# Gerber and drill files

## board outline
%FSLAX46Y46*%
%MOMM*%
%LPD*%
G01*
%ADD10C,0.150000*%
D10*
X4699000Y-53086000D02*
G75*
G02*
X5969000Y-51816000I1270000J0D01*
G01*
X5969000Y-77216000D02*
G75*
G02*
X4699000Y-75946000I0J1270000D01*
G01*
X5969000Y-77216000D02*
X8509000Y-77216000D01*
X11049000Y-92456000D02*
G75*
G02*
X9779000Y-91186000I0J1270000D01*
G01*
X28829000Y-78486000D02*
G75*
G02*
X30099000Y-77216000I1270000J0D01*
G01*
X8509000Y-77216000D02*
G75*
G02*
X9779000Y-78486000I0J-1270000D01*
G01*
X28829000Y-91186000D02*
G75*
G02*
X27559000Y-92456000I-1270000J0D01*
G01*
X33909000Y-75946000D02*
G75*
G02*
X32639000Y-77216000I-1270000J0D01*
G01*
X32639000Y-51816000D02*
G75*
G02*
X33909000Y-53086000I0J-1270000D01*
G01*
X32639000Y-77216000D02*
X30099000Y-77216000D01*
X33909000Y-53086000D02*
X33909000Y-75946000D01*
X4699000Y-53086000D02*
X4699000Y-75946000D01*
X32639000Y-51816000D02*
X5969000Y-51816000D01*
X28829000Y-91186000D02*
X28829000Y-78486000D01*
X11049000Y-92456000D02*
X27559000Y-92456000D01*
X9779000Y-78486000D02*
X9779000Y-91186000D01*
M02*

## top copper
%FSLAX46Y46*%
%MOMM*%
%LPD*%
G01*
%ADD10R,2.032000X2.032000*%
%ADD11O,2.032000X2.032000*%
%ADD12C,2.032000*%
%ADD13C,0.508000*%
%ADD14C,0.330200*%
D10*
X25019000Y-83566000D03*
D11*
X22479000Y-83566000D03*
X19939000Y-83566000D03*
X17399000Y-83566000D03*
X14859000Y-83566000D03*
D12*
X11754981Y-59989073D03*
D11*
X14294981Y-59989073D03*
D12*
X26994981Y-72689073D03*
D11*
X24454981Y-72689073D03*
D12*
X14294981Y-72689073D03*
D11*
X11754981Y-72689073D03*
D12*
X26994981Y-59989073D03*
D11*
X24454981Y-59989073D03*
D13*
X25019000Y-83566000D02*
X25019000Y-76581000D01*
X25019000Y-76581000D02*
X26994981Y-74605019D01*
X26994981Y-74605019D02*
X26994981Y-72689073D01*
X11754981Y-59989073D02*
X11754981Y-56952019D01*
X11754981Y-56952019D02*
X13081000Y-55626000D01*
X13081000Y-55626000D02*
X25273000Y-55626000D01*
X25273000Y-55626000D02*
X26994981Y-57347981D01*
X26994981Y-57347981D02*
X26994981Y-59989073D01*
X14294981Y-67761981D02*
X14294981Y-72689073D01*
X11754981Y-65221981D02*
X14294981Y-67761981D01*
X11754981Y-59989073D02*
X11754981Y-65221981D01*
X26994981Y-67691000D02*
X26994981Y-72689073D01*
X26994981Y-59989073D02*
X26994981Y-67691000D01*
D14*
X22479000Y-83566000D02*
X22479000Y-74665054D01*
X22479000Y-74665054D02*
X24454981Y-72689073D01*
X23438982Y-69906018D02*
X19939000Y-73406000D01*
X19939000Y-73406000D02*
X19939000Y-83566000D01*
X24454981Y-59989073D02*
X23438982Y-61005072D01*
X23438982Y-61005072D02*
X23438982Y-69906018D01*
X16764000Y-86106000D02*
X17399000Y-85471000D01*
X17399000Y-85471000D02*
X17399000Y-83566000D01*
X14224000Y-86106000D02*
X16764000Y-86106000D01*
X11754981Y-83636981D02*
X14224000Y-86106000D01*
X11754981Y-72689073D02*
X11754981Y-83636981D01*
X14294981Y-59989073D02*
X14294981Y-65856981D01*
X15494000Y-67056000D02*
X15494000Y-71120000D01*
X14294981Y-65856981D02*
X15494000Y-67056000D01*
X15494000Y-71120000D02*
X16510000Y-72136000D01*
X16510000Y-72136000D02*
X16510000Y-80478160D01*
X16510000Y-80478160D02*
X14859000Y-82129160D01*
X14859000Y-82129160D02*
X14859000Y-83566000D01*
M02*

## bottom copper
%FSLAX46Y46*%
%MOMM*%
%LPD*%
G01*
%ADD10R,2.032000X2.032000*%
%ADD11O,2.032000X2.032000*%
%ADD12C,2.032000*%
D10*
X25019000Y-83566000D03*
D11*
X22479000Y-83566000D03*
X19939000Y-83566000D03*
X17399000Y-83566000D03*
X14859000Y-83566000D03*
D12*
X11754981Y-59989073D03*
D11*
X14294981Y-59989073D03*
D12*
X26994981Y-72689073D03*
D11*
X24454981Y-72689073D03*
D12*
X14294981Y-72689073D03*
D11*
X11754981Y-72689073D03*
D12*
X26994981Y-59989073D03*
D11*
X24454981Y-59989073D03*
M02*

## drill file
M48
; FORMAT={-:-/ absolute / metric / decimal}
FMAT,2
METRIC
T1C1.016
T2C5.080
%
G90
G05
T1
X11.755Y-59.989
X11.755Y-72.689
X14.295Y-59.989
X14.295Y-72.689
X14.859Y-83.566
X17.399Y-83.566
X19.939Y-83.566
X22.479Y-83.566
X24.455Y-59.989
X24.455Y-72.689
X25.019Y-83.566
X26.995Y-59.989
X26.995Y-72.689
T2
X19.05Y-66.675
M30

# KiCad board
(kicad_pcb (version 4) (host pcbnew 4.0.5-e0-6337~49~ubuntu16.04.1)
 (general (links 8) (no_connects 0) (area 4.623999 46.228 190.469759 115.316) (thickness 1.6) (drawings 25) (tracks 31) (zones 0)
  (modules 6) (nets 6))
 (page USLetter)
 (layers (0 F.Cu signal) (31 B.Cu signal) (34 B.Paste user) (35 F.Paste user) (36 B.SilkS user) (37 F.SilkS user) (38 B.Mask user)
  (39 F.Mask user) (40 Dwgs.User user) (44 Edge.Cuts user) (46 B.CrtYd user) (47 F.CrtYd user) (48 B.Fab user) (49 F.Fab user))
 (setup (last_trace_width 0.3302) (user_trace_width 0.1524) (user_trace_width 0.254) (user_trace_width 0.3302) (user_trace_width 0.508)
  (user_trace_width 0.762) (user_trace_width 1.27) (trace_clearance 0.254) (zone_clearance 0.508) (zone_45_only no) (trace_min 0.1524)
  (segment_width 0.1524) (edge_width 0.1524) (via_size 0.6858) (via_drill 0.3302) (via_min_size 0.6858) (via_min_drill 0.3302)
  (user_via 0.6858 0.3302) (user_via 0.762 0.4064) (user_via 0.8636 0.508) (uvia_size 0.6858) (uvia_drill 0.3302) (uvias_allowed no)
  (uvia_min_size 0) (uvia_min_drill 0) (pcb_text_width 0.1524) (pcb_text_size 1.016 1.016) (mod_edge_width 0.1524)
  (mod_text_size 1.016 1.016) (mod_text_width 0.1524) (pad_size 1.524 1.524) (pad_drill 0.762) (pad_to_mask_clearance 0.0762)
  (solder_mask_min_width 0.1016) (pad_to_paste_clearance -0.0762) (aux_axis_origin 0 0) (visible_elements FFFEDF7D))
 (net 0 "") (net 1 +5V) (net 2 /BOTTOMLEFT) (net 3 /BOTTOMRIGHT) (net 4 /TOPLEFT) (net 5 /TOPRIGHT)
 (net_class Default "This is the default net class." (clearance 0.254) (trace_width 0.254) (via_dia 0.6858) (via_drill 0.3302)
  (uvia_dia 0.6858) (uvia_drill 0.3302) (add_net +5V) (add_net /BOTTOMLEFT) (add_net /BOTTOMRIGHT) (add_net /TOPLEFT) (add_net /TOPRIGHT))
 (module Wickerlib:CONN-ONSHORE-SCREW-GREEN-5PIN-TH (layer F.Cu) (at 25.019 83.566 270)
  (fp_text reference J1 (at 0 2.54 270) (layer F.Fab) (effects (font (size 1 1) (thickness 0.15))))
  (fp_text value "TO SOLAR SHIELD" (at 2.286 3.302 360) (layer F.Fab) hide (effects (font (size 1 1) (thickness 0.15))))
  (pad 1 thru_hole rect (at 0 0 270) (size 2.032 2.032) (drill 1.016) (layers *.Cu *.Mask F.SilkS) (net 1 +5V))
  (pad 2 thru_hole oval (at 0 2.54 270) (size 2.032 2.032) (drill 1.016) (layers *.Cu *.Mask F.SilkS) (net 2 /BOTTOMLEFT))
  (pad 3 thru_hole oval (at 0 5.08 270) (size 2.032 2.032) (drill 1.016) (layers *.Cu *.Mask F.SilkS) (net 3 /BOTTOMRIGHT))
  (pad 4 thru_hole oval (at 0 7.62 270) (size 2.032 2.032) (drill 1.016) (layers *.Cu *.Mask F.SilkS) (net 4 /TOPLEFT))
  (pad 5 thru_hole oval (at 0 10.16 270) (size 2.032 2.032) (drill 1.016) (layers *.Cu *.Mask F.SilkS) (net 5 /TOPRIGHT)))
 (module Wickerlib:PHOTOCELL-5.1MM (layer F.Cu) (at 13.024981 59.989073 90)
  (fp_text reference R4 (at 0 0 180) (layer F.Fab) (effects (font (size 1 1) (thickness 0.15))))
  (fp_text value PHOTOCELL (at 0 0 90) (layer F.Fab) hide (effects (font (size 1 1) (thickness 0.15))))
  (pad 1 thru_hole circle (at 0 -1.27 90) (size 2.032 2.032) (drill 1.016) (layers *.Cu *.Mask F.SilkS) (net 1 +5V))
  (pad 2 thru_hole oval (at 0 1.27 90) (size 2.032 2.032) (drill 1.016) (layers *.Cu *.Mask F.SilkS) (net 5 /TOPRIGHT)))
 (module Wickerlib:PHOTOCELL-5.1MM (layer F.Cu) (at 25.724981 72.689073 270)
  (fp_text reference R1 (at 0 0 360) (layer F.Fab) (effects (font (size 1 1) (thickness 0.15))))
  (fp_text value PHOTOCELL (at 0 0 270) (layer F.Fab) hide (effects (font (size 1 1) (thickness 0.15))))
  (pad 1 thru_hole circle (at 0 -1.27 270) (size 2.032 2.032) (drill 1.016) (layers *.Cu *.Mask F.SilkS) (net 1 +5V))
  (pad 2 thru_hole oval (at 0 1.27 270) (size 2.032 2.032) (drill 1.016) (layers *.Cu *.Mask F.SilkS) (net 2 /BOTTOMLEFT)))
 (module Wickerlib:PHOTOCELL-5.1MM (layer F.Cu) (at 13.024981 72.689073 270)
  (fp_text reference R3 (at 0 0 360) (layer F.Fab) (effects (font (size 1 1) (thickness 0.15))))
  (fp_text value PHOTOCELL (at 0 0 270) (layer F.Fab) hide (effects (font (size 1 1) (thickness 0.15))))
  (pad 1 thru_hole circle (at 0 -1.27 270) (size 2.032 2.032) (drill 1.016) (layers *.Cu *.Mask F.SilkS) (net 1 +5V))
  (pad 2 thru_hole oval (at 0 1.27 270) (size 2.032 2.032) (drill 1.016) (layers *.Cu *.Mask F.SilkS) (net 4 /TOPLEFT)))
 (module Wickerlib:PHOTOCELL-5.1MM (layer F.Cu) (at 25.724981 59.989073 270)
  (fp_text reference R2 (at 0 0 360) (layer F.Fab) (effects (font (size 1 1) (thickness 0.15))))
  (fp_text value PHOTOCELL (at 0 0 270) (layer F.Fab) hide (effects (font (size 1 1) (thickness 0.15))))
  (pad 1 thru_hole circle (at 0 -1.27 270) (size 2.032 2.032) (drill 1.016) (layers *.Cu *.Mask F.SilkS) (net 1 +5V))
  (pad 2 thru_hole oval (at 0 1.27 270) (size 2.032 2.032) (drill 1.016) (layers *.Cu *.Mask F.SilkS) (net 3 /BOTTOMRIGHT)))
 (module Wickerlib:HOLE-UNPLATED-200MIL (layer F.Cu) (at 19.05 66.675)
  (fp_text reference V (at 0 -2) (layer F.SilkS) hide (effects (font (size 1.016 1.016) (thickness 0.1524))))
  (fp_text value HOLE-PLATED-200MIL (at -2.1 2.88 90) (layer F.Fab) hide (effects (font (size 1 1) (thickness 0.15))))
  (pad "" np_thru_hole circle (at 0 0) (size 5.08 5.08) (drill 5.08) (layers *.Cu)))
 (gr_arc (start 5.969 53.086) (end 4.699 53.086) (angle 90) (layer Edge.Cuts) (width 0.15))
 (gr_arc (start 5.969 75.946) (end 5.969 77.216) (angle 90) (layer Edge.Cuts) (width 0.15))
 (gr_line (start 5.969 77.216) (end 8.509 77.216) (layer Edge.Cuts) (width 0.15))
 (gr_arc (start 11.049 91.186) (end 11.049 92.456) (angle 90) (layer Edge.Cuts) (width 0.15))
 (gr_arc (start 30.099 78.486) (end 28.829 78.486) (angle 90) (layer Edge.Cuts) (width 0.15))
 (gr_arc (start 8.509 78.486) (end 8.509 77.216) (angle 90) (layer Edge.Cuts) (width 0.15))
 (gr_arc (start 27.559 91.186) (end 28.829 91.186) (angle 90) (layer Edge.Cuts) (width 0.15))
 (gr_arc (start 32.639 75.946) (end 33.909 75.946) (angle 90) (layer Edge.Cuts) (width 0.15))
 (gr_arc (start 32.639 53.086) (end 32.639 51.816) (angle 90) (layer Edge.Cuts) (width 0.15))
 (gr_line (start 32.639 77.216) (end 30.099 77.216) (layer Edge.Cuts) (width 0.15))
 (gr_line (start 33.909 53.086) (end 33.909 75.946) (layer Edge.Cuts) (width 0.15))
 (gr_line (start 4.699 53.086) (end 4.699 75.946) (layer Edge.Cuts) (width 0.15))
 (gr_line (start 32.639 51.816) (end 5.969 51.816) (layer Edge.Cuts) (width 0.15))
 (gr_line (start 28.829 91.186) (end 28.829 78.486) (layer Edge.Cuts) (width 0.15))
 (gr_line (start 11.049 92.456) (end 27.559 92.456) (layer Edge.Cuts) (width 0.15))
 (gr_line (start 9.779 78.486) (end 9.779 91.186) (layer Edge.Cuts) (width 0.15))
 (segment (start 25.019 83.566) (end 25.019 76.581) (width 0.508) (layer F.Cu) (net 1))
 (segment (start 25.019 76.581) (end 26.994981 74.605019) (width 0.508) (layer F.Cu) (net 1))
 (segment (start 26.994981 74.605019) (end 26.994981 72.689073) (width 0.508) (layer F.Cu) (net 1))
 (segment (start 11.754981 59.989073) (end 11.754981 56.952019) (width 0.508) (layer F.Cu) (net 1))
 (segment (start 11.754981 56.952019) (end 13.081 55.626) (width 0.508) (layer F.Cu) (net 1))
 (segment (start 13.081 55.626) (end 25.273 55.626) (width 0.508) (layer F.Cu) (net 1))
 (segment (start 25.273 55.626) (end 26.994981 57.347981) (width 0.508) (layer F.Cu) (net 1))
 (segment (start 26.994981 57.347981) (end 26.994981 59.989073) (width 0.508) (layer F.Cu) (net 1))
 (segment (start 14.294981 67.761981) (end 14.294981 72.689073) (width 0.508) (layer F.Cu) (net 1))
 (segment (start 11.754981 65.221981) (end 14.294981 67.761981) (width 0.508) (layer F.Cu) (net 1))
 (segment (start 11.754981 59.989073) (end 11.754981 65.221981) (width 0.508) (layer F.Cu) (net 1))
 (segment (start 26.994981 67.691) (end 26.994981 72.689073) (width 0.508) (layer F.Cu) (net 1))
 (segment (start 26.994981 59.989073) (end 26.994981 67.691) (width 0.508) (layer F.Cu) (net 1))
 (segment (start 22.479 83.566) (end 22.479 74.665054) (width 0.3302) (layer F.Cu) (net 2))
 (segment (start 22.479 74.665054) (end 24.454981 72.689073) (width 0.3302) (layer F.Cu) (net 2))
 (segment (start 23.438982 69.906018) (end 19.939 73.406) (width 0.3302) (layer F.Cu) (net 3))
 (segment (start 19.939 73.406) (end 19.939 83.566) (width 0.3302) (layer F.Cu) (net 3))
 (segment (start 24.454981 59.989073) (end 23.438982 61.005072) (width 0.3302) (layer F.Cu) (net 3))
 (segment (start 23.438982 61.005072) (end 23.438982 69.906018) (width 0.3302) (layer F.Cu) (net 3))
 (segment (start 16.764 86.106) (end 17.399 85.471) (width 0.3302) (layer F.Cu) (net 4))
 (segment (start 17.399 85.471) (end 17.399 83.566) (width 0.3302) (layer F.Cu) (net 4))
 (segment (start 14.224 86.106) (end 16.764 86.106) (width 0.3302) (layer F.Cu) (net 4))
 (segment (start 11.754981 83.636981) (end 14.224 86.106) (width 0.3302) (layer F.Cu) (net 4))
 (segment (start 11.754981 72.689073) (end 11.754981 83.636981) (width 0.3302) (layer F.Cu) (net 4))
 (segment (start 14.294981 59.989073) (end 14.294981 65.856981) (width 0.3302) (layer F.Cu) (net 5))
 (segment (start 15.494 67.056) (end 15.494 71.12) (width 0.3302) (layer F.Cu) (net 5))
 (segment (start 14.294981 65.856981) (end 15.494 67.056) (width 0.3302) (layer F.Cu) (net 5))
 (segment (start 15.494 71.12) (end 16.51 72.136) (width 0.3302) (layer F.Cu) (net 5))
 (segment (start 16.51 72.136) (end 16.51 80.47816) (width 0.3302) (layer F.Cu) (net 5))
 (segment (start 16.51 80.47816) (end 14.859 82.12916) (width 0.3302) (layer F.Cu) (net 5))
 (segment (start 14.859 82.12916) (end 14.859 83.566) (width 0.3302) (layer F.Cu) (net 5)))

